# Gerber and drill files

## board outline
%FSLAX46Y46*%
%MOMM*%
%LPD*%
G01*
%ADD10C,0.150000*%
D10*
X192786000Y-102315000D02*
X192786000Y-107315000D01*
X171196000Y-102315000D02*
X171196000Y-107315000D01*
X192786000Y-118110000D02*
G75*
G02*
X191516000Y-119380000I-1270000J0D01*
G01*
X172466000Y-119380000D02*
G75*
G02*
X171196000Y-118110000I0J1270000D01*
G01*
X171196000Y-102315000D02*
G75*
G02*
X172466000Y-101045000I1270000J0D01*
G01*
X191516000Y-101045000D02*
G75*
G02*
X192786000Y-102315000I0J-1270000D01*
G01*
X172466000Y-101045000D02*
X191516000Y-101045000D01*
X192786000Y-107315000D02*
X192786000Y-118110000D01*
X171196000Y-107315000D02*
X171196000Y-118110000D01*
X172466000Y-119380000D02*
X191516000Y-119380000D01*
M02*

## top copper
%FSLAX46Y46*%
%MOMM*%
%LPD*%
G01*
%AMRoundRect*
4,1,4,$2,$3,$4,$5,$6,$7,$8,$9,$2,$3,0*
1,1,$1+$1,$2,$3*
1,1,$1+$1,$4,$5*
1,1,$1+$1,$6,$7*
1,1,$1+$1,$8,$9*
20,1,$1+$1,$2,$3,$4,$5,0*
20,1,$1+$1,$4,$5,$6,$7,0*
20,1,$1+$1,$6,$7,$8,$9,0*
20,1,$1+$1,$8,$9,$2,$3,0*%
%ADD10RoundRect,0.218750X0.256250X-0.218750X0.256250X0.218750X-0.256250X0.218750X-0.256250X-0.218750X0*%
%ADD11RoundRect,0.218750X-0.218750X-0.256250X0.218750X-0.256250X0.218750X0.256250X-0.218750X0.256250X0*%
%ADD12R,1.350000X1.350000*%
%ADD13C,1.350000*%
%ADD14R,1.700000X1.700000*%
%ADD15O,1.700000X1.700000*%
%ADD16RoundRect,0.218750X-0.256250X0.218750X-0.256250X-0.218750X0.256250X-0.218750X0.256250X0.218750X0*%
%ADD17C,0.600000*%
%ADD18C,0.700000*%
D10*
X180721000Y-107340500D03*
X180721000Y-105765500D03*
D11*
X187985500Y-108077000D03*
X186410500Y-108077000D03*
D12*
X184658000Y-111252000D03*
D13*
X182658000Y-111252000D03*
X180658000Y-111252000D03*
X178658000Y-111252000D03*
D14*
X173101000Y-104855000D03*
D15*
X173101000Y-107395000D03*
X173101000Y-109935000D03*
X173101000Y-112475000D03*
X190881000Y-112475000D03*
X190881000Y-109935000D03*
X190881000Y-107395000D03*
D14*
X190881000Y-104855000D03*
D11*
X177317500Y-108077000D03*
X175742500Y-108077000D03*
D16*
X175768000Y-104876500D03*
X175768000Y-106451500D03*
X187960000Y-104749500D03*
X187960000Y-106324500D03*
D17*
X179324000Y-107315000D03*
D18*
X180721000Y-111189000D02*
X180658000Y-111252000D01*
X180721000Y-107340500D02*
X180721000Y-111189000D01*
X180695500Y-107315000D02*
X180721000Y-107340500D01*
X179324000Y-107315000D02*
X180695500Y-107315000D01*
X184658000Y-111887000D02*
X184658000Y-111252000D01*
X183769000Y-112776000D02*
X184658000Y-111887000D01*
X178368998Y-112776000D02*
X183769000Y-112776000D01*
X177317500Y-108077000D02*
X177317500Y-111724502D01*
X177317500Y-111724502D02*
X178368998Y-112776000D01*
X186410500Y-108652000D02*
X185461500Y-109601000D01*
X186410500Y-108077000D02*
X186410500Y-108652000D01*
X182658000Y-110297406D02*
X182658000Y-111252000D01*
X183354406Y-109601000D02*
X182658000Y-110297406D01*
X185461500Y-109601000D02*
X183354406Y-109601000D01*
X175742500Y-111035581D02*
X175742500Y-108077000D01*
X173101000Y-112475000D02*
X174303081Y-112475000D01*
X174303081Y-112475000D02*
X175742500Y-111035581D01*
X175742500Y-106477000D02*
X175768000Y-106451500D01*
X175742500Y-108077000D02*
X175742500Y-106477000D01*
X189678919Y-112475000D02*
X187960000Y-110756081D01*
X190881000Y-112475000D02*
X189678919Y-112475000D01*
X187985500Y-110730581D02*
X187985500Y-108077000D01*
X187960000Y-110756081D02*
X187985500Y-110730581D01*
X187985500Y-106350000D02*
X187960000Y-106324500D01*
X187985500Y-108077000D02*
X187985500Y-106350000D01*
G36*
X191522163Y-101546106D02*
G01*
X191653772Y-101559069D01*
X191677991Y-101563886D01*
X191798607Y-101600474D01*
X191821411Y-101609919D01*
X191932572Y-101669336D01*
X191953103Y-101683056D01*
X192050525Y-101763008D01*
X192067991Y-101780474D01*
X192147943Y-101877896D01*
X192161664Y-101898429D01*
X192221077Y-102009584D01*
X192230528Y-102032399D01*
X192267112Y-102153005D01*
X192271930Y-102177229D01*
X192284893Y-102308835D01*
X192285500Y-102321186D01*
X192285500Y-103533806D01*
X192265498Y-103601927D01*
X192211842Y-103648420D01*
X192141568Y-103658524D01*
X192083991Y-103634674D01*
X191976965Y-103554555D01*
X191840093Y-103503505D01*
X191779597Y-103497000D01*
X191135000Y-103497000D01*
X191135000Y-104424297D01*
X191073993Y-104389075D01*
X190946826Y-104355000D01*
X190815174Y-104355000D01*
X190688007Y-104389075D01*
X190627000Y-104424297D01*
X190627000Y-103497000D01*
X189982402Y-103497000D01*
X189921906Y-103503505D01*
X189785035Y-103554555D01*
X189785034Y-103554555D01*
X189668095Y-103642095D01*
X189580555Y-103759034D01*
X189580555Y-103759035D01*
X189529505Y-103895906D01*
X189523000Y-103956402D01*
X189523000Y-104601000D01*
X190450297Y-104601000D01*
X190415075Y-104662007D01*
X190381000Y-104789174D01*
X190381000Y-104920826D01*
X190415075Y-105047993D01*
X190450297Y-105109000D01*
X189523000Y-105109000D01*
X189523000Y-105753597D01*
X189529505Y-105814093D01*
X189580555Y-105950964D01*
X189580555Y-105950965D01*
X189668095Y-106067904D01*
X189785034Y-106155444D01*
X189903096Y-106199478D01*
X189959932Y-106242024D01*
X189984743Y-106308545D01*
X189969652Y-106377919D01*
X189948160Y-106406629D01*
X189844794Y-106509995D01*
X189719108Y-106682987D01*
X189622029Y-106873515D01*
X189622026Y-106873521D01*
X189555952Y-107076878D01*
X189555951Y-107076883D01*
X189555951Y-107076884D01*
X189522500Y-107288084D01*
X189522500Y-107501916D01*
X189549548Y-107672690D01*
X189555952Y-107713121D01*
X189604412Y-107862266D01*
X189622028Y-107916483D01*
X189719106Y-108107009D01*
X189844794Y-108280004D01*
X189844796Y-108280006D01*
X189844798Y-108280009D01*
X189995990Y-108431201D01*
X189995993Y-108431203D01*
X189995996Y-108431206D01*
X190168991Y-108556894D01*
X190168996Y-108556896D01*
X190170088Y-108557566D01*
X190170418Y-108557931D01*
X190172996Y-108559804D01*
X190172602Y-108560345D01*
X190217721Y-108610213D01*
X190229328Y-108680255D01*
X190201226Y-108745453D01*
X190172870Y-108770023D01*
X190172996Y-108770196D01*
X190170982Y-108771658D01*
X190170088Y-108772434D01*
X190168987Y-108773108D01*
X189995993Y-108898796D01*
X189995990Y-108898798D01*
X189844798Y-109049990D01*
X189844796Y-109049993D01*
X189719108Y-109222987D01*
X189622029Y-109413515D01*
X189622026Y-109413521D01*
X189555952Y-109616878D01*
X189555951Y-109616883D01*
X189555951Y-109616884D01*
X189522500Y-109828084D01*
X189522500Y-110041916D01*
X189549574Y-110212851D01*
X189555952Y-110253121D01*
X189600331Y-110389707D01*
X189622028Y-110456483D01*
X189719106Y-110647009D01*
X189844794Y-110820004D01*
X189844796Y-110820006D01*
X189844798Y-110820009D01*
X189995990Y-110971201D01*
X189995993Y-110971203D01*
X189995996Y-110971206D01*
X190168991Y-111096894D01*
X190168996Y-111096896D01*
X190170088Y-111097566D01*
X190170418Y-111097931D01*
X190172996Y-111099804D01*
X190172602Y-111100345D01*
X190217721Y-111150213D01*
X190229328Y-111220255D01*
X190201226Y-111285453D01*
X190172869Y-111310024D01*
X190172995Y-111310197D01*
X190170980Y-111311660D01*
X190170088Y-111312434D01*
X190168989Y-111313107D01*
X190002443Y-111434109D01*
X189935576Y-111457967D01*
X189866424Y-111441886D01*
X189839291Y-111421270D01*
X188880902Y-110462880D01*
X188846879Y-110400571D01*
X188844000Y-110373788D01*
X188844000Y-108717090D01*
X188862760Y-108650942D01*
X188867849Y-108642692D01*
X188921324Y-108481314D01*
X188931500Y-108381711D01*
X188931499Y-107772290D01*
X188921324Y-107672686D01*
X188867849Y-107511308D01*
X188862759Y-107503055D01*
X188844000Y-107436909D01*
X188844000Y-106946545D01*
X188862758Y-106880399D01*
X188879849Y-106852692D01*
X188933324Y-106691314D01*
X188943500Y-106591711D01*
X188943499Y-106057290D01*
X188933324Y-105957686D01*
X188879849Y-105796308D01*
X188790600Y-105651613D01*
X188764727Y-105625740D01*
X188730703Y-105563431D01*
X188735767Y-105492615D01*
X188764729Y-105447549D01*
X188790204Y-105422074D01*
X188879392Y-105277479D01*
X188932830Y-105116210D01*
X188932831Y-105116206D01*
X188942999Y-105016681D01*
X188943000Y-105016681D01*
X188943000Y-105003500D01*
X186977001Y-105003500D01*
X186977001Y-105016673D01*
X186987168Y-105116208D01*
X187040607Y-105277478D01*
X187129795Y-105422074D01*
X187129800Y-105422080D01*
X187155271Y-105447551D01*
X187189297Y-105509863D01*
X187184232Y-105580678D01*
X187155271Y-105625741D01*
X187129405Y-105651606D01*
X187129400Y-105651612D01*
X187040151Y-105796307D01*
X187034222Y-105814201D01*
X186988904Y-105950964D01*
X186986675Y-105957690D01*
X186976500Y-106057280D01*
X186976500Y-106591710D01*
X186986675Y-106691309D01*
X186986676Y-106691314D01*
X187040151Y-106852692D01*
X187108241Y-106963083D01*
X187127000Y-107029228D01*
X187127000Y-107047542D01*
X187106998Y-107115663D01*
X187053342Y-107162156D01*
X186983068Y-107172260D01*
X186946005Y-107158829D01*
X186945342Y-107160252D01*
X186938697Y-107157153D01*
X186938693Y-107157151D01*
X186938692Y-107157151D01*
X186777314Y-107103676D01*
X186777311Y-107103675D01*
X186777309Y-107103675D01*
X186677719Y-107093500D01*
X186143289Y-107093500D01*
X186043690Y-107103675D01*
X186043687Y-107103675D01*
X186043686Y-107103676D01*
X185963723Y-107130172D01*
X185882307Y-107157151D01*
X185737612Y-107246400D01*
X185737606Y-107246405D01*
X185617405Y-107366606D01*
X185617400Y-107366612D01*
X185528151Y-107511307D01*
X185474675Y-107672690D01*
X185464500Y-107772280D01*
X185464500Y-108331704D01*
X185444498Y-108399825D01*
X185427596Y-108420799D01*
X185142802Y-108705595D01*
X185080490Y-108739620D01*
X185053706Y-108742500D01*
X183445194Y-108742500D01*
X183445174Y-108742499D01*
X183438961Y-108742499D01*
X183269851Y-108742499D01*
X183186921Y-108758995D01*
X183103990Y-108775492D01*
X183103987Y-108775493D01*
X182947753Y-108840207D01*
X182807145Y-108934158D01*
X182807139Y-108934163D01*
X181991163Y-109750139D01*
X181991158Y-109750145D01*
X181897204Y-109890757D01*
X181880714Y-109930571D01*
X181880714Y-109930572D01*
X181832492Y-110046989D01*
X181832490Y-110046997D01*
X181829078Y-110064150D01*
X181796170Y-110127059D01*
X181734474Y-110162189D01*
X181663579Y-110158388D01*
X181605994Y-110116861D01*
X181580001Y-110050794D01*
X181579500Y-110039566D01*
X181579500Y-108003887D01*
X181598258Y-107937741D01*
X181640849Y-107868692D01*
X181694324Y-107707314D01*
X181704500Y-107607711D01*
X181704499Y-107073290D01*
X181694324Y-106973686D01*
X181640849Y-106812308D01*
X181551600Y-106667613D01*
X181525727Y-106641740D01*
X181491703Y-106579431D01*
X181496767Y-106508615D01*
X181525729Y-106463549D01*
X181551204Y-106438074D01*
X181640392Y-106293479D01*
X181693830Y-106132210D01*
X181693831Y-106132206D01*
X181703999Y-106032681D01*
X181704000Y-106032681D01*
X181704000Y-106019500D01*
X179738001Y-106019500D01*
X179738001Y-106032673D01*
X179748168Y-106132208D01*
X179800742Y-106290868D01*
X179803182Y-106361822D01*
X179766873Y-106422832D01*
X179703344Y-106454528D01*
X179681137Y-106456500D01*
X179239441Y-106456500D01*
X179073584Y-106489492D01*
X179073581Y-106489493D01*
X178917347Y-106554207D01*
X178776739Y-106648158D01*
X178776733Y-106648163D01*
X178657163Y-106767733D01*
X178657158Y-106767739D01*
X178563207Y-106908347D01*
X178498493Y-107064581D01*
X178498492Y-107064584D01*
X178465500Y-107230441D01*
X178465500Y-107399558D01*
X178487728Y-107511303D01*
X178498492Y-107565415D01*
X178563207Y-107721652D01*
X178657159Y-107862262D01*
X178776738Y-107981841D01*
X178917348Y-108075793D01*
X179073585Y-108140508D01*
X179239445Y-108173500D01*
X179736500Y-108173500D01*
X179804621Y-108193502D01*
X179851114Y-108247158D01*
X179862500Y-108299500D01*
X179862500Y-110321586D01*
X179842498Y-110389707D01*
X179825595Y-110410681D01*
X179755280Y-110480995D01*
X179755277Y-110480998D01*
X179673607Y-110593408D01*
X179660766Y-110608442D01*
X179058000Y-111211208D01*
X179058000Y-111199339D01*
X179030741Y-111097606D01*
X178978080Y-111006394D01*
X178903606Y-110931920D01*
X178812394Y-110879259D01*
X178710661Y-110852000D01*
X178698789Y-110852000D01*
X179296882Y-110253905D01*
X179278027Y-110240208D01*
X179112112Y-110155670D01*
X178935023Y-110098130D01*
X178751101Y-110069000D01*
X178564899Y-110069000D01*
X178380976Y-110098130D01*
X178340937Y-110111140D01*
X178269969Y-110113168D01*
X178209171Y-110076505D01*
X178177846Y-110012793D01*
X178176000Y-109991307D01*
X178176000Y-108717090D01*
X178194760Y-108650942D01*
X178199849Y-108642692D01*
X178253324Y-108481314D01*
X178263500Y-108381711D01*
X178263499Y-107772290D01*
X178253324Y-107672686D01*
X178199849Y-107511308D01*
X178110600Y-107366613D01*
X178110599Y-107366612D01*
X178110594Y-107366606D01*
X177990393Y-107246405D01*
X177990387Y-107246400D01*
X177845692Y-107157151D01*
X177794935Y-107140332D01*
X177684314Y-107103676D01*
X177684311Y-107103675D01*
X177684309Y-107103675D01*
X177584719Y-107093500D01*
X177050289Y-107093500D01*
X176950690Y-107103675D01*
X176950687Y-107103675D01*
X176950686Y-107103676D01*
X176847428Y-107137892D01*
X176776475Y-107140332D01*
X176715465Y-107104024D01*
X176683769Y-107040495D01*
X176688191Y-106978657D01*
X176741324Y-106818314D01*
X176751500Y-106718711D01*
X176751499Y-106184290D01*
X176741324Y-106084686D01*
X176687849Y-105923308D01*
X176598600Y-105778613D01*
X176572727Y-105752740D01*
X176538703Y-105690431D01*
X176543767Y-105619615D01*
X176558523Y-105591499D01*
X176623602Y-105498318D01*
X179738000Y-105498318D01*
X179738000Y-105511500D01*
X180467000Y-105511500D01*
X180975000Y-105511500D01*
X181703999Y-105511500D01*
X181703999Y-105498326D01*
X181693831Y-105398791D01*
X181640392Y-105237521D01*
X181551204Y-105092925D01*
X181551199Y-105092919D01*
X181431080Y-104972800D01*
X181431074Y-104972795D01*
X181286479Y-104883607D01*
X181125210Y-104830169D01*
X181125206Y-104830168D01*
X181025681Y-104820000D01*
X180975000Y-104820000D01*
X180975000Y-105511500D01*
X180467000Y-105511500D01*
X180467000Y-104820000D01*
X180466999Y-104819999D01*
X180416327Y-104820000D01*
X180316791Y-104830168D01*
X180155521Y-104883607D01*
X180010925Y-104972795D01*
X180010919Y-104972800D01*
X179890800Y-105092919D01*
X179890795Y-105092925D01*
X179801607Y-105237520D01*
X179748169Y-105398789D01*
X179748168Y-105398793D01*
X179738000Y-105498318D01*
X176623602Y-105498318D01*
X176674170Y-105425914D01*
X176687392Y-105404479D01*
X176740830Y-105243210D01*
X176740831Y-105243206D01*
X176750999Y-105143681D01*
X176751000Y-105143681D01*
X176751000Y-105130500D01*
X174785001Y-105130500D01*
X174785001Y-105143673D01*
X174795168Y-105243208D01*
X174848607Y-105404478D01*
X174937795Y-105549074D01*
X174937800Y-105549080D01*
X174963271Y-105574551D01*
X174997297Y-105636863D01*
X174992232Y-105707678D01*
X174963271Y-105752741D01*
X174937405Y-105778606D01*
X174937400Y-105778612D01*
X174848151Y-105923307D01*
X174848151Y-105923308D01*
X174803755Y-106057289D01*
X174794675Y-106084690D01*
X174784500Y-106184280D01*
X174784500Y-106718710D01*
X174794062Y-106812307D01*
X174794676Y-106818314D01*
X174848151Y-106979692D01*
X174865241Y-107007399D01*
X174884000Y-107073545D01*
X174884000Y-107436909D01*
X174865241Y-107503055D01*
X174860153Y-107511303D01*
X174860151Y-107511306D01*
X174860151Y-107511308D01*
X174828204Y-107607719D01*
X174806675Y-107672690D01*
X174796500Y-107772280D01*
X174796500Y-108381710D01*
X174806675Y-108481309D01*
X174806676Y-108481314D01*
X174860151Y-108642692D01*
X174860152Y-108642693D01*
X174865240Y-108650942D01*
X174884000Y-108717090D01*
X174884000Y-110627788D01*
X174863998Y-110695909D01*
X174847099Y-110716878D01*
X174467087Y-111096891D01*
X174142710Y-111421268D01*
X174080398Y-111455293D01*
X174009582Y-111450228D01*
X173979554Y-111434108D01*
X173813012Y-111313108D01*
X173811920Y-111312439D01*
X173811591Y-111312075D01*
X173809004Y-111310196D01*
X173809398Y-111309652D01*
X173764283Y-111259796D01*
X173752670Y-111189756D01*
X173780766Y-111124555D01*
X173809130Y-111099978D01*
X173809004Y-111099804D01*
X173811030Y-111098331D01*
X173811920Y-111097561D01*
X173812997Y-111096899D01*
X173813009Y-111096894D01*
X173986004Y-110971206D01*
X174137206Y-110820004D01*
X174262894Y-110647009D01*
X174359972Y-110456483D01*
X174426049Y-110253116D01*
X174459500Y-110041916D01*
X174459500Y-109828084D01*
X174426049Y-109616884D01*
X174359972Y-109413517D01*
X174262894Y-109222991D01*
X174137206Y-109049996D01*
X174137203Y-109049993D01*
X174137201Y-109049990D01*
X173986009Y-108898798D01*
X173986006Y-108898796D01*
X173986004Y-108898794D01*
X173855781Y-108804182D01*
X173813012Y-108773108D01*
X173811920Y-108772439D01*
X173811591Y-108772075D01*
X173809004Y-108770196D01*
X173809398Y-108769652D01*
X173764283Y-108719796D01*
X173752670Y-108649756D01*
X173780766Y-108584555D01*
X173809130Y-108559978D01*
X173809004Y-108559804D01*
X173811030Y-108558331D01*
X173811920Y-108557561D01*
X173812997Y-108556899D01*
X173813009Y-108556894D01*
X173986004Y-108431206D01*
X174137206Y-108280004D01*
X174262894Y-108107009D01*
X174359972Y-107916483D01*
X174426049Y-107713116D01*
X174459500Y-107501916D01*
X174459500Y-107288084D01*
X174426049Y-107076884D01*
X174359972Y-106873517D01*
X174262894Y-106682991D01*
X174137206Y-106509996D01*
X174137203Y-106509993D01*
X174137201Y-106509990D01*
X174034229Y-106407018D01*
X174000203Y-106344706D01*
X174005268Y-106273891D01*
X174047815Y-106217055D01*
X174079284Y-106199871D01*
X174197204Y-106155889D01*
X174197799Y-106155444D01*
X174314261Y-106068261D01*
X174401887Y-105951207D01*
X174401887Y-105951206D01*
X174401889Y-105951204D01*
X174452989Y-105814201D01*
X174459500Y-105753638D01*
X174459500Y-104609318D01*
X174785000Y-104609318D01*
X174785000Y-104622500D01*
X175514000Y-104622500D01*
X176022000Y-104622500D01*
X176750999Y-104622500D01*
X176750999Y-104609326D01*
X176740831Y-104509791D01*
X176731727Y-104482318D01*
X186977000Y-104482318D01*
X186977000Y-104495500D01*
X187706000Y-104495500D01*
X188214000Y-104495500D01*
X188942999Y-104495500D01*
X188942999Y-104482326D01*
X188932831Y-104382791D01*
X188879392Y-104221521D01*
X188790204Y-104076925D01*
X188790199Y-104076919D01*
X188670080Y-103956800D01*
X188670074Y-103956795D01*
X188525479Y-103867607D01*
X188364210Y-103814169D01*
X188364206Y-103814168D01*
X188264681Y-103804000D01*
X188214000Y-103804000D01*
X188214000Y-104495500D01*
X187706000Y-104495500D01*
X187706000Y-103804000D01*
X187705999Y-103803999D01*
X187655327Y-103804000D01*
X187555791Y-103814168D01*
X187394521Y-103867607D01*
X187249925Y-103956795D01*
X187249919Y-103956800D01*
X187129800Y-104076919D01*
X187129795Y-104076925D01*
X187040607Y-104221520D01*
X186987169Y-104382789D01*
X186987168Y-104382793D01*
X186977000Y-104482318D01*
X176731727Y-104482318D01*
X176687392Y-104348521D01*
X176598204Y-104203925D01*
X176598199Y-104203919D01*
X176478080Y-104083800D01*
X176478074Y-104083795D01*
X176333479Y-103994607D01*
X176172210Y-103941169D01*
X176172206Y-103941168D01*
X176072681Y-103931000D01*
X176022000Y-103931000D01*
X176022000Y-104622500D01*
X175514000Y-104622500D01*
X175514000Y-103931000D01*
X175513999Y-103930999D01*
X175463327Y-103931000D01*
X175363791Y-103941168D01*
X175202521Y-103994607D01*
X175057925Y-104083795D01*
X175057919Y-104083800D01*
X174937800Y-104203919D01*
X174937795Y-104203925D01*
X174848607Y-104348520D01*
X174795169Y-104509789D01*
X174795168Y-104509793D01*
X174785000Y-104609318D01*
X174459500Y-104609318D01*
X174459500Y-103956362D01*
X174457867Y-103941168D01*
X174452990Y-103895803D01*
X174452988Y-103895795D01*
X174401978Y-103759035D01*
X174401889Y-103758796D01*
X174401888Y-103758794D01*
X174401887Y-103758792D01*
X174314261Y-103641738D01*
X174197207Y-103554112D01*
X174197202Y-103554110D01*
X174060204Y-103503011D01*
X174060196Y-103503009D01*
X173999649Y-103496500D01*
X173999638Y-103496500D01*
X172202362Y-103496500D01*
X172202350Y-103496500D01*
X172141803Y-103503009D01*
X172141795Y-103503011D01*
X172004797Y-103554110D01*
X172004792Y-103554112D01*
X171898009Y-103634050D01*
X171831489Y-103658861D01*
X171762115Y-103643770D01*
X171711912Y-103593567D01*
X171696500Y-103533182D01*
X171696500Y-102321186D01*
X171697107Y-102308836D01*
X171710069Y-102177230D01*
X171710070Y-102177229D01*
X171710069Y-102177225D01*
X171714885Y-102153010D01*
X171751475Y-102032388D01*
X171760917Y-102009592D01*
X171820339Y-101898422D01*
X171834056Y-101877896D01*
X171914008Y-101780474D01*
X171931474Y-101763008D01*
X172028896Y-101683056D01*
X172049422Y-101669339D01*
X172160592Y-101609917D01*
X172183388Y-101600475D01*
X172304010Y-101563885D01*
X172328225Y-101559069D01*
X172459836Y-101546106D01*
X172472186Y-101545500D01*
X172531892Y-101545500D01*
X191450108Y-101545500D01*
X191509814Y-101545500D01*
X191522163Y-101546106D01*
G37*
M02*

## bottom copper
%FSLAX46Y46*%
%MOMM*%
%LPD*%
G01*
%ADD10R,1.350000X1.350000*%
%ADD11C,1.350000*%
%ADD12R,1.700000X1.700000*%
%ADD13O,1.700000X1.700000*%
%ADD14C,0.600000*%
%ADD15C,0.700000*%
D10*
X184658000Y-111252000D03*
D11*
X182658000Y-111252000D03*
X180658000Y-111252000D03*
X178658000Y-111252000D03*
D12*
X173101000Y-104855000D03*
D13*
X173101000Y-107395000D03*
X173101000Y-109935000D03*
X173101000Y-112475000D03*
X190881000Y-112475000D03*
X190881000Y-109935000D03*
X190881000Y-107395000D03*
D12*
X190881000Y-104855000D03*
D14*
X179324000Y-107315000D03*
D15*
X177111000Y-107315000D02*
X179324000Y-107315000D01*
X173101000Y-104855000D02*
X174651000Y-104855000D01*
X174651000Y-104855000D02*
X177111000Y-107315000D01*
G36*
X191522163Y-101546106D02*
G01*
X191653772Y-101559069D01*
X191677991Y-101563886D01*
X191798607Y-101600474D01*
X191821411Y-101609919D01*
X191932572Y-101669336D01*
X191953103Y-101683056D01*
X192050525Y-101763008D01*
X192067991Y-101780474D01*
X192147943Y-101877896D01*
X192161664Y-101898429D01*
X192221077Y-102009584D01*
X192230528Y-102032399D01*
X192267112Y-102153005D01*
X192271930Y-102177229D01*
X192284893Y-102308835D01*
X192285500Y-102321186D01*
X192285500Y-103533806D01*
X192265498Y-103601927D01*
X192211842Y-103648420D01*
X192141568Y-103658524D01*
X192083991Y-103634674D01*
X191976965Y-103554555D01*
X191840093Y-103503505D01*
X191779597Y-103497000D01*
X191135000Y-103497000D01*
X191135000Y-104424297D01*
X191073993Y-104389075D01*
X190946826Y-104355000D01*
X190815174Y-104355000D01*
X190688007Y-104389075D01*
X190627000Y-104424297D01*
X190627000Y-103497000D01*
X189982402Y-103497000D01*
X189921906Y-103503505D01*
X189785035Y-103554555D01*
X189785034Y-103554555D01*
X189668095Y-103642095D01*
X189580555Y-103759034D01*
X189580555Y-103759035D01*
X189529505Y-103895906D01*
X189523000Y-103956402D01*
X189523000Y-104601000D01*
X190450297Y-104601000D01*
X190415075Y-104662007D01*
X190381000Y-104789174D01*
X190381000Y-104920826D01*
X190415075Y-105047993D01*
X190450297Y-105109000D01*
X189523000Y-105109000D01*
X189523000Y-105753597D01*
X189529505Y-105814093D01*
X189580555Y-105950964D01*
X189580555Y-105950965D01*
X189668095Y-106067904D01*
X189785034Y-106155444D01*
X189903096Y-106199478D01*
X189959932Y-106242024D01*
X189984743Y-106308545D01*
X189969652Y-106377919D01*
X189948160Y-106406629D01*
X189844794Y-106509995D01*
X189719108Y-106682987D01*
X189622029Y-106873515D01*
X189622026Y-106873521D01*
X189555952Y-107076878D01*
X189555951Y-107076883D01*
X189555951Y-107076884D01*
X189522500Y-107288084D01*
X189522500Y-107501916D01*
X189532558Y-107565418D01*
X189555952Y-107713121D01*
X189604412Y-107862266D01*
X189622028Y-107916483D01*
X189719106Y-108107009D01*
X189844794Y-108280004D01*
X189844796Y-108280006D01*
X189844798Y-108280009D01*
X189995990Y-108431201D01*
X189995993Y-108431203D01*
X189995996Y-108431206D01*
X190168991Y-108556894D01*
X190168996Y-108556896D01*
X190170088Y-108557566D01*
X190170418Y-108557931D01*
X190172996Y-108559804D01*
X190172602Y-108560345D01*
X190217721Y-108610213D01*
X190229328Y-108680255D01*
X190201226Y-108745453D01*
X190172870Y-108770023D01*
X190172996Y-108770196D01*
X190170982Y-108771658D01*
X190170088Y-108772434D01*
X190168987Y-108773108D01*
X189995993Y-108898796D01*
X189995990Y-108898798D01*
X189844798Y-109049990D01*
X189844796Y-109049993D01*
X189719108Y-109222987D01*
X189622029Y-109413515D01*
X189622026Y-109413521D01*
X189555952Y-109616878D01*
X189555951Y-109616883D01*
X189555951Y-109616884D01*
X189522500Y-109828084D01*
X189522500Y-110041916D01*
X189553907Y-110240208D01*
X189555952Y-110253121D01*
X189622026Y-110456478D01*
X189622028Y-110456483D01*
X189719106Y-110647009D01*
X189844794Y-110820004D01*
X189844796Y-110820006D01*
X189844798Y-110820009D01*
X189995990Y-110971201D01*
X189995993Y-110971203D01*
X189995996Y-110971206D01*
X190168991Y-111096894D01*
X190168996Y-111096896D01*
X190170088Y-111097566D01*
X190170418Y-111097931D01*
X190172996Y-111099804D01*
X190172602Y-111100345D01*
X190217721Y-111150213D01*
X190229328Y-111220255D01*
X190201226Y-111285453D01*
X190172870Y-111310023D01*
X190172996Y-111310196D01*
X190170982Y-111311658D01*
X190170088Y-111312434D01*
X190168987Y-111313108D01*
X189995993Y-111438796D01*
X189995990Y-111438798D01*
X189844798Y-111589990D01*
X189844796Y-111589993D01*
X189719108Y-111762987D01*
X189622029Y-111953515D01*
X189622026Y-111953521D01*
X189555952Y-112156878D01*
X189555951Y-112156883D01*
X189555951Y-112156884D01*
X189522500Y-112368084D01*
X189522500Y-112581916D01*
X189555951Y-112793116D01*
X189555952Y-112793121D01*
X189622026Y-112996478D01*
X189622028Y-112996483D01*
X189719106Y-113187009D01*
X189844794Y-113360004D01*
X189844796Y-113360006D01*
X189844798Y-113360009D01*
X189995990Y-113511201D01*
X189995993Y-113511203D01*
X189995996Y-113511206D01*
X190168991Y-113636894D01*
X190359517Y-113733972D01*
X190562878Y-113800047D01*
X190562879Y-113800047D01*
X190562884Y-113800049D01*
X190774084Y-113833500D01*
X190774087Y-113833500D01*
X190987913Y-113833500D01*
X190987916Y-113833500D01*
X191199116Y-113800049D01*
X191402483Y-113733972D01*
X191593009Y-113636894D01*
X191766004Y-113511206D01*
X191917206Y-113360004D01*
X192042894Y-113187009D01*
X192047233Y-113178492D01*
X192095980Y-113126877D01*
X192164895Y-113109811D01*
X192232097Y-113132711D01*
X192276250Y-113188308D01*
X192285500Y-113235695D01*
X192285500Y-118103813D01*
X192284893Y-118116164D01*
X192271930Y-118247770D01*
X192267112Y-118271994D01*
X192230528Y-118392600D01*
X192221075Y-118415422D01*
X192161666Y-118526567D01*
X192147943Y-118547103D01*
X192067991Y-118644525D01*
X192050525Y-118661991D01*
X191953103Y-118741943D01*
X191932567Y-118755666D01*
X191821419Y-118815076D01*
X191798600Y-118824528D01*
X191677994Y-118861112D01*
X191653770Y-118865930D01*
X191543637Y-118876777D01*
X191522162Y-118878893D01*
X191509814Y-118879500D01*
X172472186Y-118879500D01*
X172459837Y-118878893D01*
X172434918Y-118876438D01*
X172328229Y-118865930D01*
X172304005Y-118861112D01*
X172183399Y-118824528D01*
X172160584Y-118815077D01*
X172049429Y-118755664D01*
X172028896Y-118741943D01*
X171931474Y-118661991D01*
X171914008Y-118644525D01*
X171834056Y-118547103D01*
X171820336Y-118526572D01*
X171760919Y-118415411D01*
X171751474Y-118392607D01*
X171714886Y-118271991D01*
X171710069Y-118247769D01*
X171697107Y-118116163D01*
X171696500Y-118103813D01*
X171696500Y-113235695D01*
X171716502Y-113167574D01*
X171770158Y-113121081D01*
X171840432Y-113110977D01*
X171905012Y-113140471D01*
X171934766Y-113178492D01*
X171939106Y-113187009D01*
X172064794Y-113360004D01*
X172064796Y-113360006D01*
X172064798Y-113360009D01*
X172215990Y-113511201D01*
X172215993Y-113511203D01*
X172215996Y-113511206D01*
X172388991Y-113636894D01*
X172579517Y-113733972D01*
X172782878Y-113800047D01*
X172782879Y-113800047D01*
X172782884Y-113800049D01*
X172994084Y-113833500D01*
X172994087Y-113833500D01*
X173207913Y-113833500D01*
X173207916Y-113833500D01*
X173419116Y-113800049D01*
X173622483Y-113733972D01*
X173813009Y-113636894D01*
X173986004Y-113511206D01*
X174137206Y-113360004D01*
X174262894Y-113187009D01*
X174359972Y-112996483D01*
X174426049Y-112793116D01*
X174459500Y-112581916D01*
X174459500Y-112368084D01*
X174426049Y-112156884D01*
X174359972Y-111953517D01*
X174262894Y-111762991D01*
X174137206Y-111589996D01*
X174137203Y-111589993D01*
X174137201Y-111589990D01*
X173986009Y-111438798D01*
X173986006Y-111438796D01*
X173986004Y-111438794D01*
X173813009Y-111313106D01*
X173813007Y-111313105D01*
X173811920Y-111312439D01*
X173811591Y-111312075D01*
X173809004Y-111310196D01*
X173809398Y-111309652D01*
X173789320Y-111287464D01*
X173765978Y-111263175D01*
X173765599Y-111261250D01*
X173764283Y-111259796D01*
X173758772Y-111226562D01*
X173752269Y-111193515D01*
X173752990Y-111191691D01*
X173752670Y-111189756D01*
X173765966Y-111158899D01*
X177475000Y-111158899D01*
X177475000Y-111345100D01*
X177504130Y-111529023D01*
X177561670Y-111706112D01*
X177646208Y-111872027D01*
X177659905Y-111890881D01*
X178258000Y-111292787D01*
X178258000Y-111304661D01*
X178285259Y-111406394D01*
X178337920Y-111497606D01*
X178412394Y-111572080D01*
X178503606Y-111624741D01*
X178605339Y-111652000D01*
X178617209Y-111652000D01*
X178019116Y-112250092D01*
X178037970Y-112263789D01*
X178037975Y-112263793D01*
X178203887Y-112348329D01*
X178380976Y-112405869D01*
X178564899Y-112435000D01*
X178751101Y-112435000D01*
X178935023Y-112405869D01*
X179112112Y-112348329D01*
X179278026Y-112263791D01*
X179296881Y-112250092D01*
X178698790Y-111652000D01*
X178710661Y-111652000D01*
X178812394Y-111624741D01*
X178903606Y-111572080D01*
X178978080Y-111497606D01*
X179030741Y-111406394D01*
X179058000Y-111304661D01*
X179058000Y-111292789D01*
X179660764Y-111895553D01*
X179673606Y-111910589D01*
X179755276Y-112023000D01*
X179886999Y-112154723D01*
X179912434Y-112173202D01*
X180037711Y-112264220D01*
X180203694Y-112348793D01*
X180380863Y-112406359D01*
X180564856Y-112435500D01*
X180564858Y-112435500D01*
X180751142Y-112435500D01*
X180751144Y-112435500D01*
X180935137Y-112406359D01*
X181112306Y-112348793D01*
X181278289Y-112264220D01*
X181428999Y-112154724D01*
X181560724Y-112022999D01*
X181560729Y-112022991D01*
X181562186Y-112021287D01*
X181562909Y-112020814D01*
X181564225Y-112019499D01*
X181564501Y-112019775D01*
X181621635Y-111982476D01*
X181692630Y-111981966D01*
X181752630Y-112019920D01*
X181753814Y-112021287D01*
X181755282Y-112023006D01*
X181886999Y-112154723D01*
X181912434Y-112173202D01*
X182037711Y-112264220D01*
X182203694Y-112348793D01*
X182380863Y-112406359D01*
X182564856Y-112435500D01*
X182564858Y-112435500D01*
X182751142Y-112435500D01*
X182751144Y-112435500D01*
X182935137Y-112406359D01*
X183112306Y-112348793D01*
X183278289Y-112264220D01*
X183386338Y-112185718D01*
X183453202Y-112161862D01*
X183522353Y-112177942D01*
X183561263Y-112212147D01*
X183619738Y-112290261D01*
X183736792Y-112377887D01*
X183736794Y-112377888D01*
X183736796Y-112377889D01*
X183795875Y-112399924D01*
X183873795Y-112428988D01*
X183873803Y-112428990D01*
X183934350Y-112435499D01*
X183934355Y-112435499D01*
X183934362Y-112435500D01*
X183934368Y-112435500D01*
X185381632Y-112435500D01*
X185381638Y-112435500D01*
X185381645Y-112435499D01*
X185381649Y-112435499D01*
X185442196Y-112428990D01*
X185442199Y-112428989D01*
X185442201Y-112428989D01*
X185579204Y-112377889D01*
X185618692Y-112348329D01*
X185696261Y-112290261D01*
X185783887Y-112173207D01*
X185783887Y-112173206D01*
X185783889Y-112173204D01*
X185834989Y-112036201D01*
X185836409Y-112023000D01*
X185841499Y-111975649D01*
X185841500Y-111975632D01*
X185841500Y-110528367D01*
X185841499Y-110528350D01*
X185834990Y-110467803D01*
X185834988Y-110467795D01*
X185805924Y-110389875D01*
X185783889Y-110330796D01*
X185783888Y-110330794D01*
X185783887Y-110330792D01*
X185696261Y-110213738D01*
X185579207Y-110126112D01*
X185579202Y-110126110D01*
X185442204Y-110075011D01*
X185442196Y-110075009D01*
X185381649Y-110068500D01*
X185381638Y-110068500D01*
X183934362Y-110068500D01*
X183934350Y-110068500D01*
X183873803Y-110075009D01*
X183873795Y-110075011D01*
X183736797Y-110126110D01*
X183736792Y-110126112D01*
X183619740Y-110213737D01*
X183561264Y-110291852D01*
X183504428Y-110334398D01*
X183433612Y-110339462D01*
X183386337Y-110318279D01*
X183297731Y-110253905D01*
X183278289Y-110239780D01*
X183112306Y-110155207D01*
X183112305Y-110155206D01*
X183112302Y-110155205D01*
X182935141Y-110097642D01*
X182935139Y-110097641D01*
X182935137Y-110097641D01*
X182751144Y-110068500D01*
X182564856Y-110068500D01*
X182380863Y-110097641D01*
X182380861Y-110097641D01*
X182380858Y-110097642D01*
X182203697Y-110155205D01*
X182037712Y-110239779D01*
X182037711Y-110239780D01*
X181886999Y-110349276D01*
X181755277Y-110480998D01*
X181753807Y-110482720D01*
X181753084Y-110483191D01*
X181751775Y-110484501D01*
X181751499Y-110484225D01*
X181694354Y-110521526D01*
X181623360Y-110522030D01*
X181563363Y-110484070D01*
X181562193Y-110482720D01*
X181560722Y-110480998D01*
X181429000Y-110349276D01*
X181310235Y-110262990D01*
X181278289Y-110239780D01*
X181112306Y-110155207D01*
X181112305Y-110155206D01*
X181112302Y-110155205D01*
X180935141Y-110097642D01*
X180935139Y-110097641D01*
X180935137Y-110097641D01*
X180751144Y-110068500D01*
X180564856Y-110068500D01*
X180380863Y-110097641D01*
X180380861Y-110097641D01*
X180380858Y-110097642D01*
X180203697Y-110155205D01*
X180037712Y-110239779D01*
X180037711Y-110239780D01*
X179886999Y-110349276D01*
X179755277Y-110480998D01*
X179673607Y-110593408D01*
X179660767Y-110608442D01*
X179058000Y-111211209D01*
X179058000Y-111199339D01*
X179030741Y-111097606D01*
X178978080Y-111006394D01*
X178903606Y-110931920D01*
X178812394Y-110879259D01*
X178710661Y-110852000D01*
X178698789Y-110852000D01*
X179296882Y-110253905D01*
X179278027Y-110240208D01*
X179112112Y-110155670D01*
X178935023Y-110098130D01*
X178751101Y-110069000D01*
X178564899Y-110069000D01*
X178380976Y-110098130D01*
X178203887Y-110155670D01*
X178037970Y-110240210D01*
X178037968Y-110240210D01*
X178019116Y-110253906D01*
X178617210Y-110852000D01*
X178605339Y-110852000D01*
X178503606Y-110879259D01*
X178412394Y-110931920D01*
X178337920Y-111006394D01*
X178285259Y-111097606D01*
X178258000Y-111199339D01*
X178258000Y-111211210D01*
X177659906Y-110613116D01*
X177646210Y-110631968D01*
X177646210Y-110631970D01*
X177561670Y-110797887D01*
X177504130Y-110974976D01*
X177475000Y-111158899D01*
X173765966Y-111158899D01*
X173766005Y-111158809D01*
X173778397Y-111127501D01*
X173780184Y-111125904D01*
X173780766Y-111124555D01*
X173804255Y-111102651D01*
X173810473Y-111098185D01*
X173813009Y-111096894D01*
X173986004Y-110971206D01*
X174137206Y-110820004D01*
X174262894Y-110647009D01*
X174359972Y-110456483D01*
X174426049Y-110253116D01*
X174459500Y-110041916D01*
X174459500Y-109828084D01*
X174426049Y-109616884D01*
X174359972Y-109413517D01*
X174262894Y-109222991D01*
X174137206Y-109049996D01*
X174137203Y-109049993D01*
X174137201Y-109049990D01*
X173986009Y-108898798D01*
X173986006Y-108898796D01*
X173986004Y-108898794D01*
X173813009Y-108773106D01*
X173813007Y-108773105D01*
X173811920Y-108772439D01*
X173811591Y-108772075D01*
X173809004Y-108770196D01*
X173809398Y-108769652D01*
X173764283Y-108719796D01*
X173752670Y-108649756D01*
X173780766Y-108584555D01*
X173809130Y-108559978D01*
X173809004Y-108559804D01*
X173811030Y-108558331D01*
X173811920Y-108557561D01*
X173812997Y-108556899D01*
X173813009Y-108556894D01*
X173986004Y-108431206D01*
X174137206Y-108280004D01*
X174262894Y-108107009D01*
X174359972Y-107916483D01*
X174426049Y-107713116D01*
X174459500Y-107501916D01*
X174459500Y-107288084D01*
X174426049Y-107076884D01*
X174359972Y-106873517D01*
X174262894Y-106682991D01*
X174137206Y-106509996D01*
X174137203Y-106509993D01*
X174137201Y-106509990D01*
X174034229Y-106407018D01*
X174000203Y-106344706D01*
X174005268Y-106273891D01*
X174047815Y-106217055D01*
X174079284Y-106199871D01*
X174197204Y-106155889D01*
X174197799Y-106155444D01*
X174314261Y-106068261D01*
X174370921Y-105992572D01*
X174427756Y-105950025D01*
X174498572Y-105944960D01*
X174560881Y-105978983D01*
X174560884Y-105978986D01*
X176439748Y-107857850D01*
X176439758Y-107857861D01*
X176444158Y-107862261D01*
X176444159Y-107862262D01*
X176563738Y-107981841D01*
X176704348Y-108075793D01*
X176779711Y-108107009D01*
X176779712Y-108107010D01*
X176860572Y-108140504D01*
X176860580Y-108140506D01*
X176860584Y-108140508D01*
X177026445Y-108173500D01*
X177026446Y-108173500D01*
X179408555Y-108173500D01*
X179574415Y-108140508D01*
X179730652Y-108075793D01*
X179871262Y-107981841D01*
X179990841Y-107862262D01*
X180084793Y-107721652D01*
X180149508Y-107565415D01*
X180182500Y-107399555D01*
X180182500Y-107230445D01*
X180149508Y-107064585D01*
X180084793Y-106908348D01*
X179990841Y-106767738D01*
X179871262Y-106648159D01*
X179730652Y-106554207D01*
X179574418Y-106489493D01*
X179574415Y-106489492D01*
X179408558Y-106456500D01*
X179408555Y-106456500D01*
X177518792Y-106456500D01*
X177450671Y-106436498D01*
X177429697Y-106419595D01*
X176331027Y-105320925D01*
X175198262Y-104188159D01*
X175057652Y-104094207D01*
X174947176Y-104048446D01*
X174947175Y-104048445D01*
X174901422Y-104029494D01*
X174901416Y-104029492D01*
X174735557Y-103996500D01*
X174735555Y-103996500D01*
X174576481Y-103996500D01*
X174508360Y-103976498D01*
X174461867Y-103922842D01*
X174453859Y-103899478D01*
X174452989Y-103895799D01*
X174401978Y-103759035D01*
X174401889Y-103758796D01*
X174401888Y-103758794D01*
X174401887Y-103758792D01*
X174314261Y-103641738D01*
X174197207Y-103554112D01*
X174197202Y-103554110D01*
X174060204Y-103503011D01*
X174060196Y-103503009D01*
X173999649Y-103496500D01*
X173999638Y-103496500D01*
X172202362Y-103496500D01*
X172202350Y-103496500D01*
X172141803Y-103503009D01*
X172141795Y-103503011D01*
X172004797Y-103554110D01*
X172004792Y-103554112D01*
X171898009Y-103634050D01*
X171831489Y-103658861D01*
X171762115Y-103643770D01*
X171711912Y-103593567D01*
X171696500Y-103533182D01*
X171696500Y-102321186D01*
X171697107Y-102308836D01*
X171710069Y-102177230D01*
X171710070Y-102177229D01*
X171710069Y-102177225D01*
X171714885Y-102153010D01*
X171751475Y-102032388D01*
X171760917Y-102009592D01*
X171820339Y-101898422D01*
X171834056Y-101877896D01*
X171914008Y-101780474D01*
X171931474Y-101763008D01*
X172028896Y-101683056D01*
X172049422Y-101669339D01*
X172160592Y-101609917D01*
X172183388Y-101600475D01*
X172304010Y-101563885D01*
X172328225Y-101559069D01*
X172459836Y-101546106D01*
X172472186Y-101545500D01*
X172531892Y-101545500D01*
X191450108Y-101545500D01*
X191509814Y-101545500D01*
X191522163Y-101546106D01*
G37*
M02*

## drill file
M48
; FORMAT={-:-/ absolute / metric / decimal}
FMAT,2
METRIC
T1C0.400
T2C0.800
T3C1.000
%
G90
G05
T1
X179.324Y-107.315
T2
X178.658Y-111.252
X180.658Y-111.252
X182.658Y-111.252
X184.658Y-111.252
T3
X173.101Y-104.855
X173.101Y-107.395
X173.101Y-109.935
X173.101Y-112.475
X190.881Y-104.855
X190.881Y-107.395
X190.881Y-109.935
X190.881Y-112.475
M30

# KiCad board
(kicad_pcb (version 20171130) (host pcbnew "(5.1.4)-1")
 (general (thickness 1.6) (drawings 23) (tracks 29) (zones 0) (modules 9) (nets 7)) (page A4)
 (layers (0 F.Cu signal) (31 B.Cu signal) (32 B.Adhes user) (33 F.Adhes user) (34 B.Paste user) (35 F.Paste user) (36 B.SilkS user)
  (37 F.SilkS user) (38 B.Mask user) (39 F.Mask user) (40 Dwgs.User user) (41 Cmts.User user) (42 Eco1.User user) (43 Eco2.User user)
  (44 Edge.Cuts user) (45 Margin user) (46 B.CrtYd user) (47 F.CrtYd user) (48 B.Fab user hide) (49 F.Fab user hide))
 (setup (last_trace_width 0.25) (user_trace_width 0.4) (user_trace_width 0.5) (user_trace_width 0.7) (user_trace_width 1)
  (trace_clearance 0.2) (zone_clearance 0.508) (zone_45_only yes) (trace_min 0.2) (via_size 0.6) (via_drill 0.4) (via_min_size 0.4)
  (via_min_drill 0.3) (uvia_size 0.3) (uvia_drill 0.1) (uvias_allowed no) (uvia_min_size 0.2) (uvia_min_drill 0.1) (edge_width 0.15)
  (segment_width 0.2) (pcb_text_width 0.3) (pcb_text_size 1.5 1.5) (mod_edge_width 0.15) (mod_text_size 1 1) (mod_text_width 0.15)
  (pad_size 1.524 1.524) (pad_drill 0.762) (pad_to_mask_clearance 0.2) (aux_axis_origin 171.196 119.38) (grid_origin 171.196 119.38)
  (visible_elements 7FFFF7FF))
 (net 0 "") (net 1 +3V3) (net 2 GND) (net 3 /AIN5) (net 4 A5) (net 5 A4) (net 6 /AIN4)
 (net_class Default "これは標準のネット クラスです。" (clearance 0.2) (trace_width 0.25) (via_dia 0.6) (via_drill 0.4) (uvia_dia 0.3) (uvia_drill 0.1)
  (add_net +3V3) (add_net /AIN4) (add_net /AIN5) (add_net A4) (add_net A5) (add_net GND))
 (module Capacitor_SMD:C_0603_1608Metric (layer F.Cu) (at 180.721 106.553 90)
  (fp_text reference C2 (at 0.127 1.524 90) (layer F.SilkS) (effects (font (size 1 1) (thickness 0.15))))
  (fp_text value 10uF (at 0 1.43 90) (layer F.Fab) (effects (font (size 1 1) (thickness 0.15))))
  (pad 1 smd roundrect (at -0.7875 0 90) (size 0.875 0.95) (layers F.Cu F.Paste F.Mask) (roundrect_rratio 0.25) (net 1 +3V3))
  (pad 2 smd roundrect (at 0.7875 0 90) (size 0.875 0.95) (layers F.Cu F.Paste F.Mask) (roundrect_rratio 0.25) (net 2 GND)))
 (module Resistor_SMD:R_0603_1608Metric (layer F.Cu) (at 187.198 108.077)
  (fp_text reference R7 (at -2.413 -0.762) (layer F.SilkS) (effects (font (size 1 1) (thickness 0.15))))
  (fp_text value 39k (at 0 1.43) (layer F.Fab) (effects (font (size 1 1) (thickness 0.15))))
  (pad 2 smd roundrect (at 0.7875 0) (size 0.875 0.95) (layers F.Cu F.Paste F.Mask) (roundrect_rratio 0.25) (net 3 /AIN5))
  (pad 1 smd roundrect (at -0.7875 0) (size 0.875 0.95) (layers F.Cu F.Paste F.Mask) (roundrect_rratio 0.25) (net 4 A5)))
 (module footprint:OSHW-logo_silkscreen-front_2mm (layer F.Cu) (at 191.262 102.315)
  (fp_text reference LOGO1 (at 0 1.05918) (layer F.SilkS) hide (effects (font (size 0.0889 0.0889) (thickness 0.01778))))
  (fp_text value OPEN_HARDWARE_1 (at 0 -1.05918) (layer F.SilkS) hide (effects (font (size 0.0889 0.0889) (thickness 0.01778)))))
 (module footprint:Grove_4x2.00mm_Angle (layer F.Cu) (at 184.658 111.252 180)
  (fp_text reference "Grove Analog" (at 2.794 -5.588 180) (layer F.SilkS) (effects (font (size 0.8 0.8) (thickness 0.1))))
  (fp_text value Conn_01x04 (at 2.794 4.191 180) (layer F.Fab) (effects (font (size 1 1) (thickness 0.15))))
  (pad 1 thru_hole rect (at 0 0 180) (size 1.35 1.35) (drill 0.8) (layers *.Cu *.Mask) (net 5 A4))
  (pad 2 thru_hole circle (at 2 0 180) (size 1.35 1.35) (drill 0.8) (layers *.Cu *.Mask) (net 4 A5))
  (pad 3 thru_hole circle (at 4 0 180) (size 1.35 1.35) (drill 0.8) (layers *.Cu *.Mask) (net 1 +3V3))
  (pad 4 thru_hole circle (at 6 0 180) (size 1.35 1.35) (drill 0.8) (layers *.Cu *.Mask) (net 2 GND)))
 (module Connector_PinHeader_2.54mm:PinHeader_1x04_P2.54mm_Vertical (layer F.Cu) (at 173.101 104.855)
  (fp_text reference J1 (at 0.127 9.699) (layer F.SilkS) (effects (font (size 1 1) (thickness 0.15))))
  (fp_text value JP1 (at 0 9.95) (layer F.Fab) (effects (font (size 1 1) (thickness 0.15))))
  (pad 1 thru_hole rect (at 0 0) (size 1.7 1.7) (drill 1) (layers *.Cu *.Mask) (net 1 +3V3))
  (pad 2 thru_hole oval (at 0 2.54) (size 1.7 1.7) (drill 1) (layers *.Cu *.Mask))
  (pad 3 thru_hole oval (at 0 5.08) (size 1.7 1.7) (drill 1) (layers *.Cu *.Mask))
  (pad 4 thru_hole oval (at 0 7.62) (size 1.7 1.7) (drill 1) (layers *.Cu *.Mask) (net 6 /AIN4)))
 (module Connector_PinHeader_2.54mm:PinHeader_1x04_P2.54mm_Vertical (layer F.Cu) (at 190.881 104.855)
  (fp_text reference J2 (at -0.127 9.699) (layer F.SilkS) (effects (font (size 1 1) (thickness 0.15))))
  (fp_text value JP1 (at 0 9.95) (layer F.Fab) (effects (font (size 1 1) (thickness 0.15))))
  (pad 4 thru_hole oval (at 0 7.62) (size 1.7 1.7) (drill 1) (layers *.Cu *.Mask) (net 3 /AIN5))
  (pad 3 thru_hole oval (at 0 5.08) (size 1.7 1.7) (drill 1) (layers *.Cu *.Mask))
  (pad 2 thru_hole oval (at 0 2.54) (size 1.7 1.7) (drill 1) (layers *.Cu *.Mask))
  (pad 1 thru_hole rect (at 0 0) (size 1.7 1.7) (drill 1) (layers *.Cu *.Mask) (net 2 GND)))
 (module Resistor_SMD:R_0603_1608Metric (layer F.Cu) (at 176.53 108.077)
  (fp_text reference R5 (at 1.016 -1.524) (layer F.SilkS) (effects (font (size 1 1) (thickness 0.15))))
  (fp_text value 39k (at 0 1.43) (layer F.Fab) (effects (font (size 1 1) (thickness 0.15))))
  (pad 2 smd roundrect (at 0.7875 0) (size 0.875 0.95) (layers F.Cu F.Paste F.Mask) (roundrect_rratio 0.25) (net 5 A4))
  (pad 1 smd roundrect (at -0.7875 0) (size 0.875 0.95) (layers F.Cu F.Paste F.Mask) (roundrect_rratio 0.25) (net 6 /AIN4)))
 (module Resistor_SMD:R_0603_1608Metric (layer F.Cu) (at 175.768 105.664 270)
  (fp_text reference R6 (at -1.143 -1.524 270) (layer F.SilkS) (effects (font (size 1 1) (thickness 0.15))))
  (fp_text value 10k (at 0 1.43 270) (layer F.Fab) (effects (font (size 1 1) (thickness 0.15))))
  (pad 1 smd roundrect (at -0.7875 0 270) (size 0.875 0.95) (layers F.Cu F.Paste F.Mask) (roundrect_rratio 0.25) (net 2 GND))
  (pad 2 smd roundrect (at 0.7875 0 270) (size 0.875 0.95) (layers F.Cu F.Paste F.Mask) (roundrect_rratio 0.25) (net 6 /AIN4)))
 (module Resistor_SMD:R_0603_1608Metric (layer F.Cu) (at 187.96 105.537 270)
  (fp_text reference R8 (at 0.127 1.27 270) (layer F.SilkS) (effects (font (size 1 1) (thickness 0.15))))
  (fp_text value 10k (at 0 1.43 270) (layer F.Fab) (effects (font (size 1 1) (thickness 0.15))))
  (pad 1 smd roundrect (at -0.7875 0 270) (size 0.875 0.95) (layers F.Cu F.Paste F.Mask) (roundrect_rratio 0.25) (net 2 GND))
  (pad 2 smd roundrect (at 0.7875 0 270) (size 0.875 0.95) (layers F.Cu F.Paste F.Mask) (roundrect_rratio 0.25) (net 3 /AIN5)))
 (gr_line (start 192.786 102.315) (end 192.786 107.315) (layer Edge.Cuts) (width 0.15))
 (gr_line (start 171.196 102.315) (end 171.196 107.315) (layer Edge.Cuts) (width 0.15))
 (gr_arc (start 191.516 118.11) (end 192.786 118.11) (angle 90) (layer Edge.Cuts) (width 0.15))
 (gr_arc (start 172.466 118.11) (end 172.466 119.38) (angle 90) (layer Edge.Cuts) (width 0.15))
 (gr_arc (start 172.466 102.315) (end 171.196 102.315) (angle 90) (layer Edge.Cuts) (width 0.15))
 (gr_arc (start 191.516 102.315) (end 191.516 101.045) (angle 90) (layer Edge.Cuts) (width 0.15))
 (gr_line (start 172.466 101.045) (end 191.516 101.045) (angle 90) (layer Edge.Cuts) (width 0.15))
 (gr_line (start 192.786 107.315) (end 192.786 118.11) (angle 90) (layer Edge.Cuts) (width 0.15))
 (gr_line (start 171.196 107.315) (end 171.196 118.11) (angle 90) (layer Edge.Cuts) (width 0.15))
 (gr_line (start 172.466 119.38) (end 191.516 119.38) (angle 90) (layer Edge.Cuts) (width 0.15))
 (segment (start 180.721 111.189) (end 180.658 111.252) (width 0.7) (layer F.Cu) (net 1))
 (segment (start 180.721 107.3405) (end 180.721 111.189) (width 0.7) (layer F.Cu) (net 1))
 (via (at 179.324 107.315) (size 0.6) (drill 0.4) (layers F.Cu B.Cu) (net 1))
 (segment (start 177.111 107.315) (end 179.324 107.315) (width 0.7) (layer B.Cu) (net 1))
 (segment (start 173.101 104.855) (end 174.651 104.855) (width 0.7) (layer B.Cu) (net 1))
 (segment (start 174.651 104.855) (end 177.111 107.315) (width 0.7) (layer B.Cu) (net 1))
 (segment (start 180.6955 107.315) (end 180.721 107.3405) (width 0.7) (layer F.Cu) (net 1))
 (segment (start 179.324 107.315) (end 180.6955 107.315) (width 0.7) (layer F.Cu) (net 1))
 (segment (start 184.658 111.887) (end 184.658 111.252) (width 0.7) (layer F.Cu) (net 5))
 (segment (start 183.769 112.776) (end 184.658 111.887) (width 0.7) (layer F.Cu) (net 5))
 (segment (start 178.368998 112.776) (end 183.769 112.776) (width 0.7) (layer F.Cu) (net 5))
 (segment (start 177.3175 108.077) (end 177.3175 111.724502) (width 0.7) (layer F.Cu) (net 5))
 (segment (start 177.3175 111.724502) (end 178.368998 112.776) (width 0.7) (layer F.Cu) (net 5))
 (segment (start 186.4105 108.652) (end 185.4615 109.601) (width 0.7) (layer F.Cu) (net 4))
 (segment (start 186.4105 108.077) (end 186.4105 108.652) (width 0.7) (layer F.Cu) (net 4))
 (segment (start 182.658 110.297406) (end 182.658 111.252) (width 0.7) (layer F.Cu) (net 4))
 (segment (start 183.354406 109.601) (end 182.658 110.297406) (width 0.7) (layer F.Cu) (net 4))
 (segment (start 185.4615 109.601) (end 183.354406 109.601) (width 0.7) (layer F.Cu) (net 4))
 (segment (start 175.7425 111.035581) (end 175.7425 108.077) (width 0.7) (layer F.Cu) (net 6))
 (segment (start 173.101 112.475) (end 174.303081 112.475) (width 0.7) (layer F.Cu) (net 6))
 (segment (start 174.303081 112.475) (end 175.7425 111.035581) (width 0.7) (layer F.Cu) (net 6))
 (segment (start 175.7425 106.477) (end 175.768 106.4515) (width 0.7) (layer F.Cu) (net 6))
 (segment (start 175.7425 108.077) (end 175.7425 106.477) (width 0.7) (layer F.Cu) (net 6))
 (segment (start 189.678919 112.475) (end 187.96 110.756081) (width 0.7) (layer F.Cu) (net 3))
 (segment (start 190.881 112.475) (end 189.678919 112.475) (width 0.7) (layer F.Cu) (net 3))
 (segment (start 187.9855 110.730581) (end 187.9855 108.077) (width 0.7) (layer F.Cu) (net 3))
 (segment (start 187.96 110.756081) (end 187.9855 110.730581) (width 0.7) (layer F.Cu) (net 3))
 (segment (start 187.9855 106.35) (end 187.96 106.3245) (width 0.7) (layer F.Cu) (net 3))
 (segment (start 187.9855 108.077) (end 187.9855 106.35) (width 0.7) (layer F.Cu) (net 3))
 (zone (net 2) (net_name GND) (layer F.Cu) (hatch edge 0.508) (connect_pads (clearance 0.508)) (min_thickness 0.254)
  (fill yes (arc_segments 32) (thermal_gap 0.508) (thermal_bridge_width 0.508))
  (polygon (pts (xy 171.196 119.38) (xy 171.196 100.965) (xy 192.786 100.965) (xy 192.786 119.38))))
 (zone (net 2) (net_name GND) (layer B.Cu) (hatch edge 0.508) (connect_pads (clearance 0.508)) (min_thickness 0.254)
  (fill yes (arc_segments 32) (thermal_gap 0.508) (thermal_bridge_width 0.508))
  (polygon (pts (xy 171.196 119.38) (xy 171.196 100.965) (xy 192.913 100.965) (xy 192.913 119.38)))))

